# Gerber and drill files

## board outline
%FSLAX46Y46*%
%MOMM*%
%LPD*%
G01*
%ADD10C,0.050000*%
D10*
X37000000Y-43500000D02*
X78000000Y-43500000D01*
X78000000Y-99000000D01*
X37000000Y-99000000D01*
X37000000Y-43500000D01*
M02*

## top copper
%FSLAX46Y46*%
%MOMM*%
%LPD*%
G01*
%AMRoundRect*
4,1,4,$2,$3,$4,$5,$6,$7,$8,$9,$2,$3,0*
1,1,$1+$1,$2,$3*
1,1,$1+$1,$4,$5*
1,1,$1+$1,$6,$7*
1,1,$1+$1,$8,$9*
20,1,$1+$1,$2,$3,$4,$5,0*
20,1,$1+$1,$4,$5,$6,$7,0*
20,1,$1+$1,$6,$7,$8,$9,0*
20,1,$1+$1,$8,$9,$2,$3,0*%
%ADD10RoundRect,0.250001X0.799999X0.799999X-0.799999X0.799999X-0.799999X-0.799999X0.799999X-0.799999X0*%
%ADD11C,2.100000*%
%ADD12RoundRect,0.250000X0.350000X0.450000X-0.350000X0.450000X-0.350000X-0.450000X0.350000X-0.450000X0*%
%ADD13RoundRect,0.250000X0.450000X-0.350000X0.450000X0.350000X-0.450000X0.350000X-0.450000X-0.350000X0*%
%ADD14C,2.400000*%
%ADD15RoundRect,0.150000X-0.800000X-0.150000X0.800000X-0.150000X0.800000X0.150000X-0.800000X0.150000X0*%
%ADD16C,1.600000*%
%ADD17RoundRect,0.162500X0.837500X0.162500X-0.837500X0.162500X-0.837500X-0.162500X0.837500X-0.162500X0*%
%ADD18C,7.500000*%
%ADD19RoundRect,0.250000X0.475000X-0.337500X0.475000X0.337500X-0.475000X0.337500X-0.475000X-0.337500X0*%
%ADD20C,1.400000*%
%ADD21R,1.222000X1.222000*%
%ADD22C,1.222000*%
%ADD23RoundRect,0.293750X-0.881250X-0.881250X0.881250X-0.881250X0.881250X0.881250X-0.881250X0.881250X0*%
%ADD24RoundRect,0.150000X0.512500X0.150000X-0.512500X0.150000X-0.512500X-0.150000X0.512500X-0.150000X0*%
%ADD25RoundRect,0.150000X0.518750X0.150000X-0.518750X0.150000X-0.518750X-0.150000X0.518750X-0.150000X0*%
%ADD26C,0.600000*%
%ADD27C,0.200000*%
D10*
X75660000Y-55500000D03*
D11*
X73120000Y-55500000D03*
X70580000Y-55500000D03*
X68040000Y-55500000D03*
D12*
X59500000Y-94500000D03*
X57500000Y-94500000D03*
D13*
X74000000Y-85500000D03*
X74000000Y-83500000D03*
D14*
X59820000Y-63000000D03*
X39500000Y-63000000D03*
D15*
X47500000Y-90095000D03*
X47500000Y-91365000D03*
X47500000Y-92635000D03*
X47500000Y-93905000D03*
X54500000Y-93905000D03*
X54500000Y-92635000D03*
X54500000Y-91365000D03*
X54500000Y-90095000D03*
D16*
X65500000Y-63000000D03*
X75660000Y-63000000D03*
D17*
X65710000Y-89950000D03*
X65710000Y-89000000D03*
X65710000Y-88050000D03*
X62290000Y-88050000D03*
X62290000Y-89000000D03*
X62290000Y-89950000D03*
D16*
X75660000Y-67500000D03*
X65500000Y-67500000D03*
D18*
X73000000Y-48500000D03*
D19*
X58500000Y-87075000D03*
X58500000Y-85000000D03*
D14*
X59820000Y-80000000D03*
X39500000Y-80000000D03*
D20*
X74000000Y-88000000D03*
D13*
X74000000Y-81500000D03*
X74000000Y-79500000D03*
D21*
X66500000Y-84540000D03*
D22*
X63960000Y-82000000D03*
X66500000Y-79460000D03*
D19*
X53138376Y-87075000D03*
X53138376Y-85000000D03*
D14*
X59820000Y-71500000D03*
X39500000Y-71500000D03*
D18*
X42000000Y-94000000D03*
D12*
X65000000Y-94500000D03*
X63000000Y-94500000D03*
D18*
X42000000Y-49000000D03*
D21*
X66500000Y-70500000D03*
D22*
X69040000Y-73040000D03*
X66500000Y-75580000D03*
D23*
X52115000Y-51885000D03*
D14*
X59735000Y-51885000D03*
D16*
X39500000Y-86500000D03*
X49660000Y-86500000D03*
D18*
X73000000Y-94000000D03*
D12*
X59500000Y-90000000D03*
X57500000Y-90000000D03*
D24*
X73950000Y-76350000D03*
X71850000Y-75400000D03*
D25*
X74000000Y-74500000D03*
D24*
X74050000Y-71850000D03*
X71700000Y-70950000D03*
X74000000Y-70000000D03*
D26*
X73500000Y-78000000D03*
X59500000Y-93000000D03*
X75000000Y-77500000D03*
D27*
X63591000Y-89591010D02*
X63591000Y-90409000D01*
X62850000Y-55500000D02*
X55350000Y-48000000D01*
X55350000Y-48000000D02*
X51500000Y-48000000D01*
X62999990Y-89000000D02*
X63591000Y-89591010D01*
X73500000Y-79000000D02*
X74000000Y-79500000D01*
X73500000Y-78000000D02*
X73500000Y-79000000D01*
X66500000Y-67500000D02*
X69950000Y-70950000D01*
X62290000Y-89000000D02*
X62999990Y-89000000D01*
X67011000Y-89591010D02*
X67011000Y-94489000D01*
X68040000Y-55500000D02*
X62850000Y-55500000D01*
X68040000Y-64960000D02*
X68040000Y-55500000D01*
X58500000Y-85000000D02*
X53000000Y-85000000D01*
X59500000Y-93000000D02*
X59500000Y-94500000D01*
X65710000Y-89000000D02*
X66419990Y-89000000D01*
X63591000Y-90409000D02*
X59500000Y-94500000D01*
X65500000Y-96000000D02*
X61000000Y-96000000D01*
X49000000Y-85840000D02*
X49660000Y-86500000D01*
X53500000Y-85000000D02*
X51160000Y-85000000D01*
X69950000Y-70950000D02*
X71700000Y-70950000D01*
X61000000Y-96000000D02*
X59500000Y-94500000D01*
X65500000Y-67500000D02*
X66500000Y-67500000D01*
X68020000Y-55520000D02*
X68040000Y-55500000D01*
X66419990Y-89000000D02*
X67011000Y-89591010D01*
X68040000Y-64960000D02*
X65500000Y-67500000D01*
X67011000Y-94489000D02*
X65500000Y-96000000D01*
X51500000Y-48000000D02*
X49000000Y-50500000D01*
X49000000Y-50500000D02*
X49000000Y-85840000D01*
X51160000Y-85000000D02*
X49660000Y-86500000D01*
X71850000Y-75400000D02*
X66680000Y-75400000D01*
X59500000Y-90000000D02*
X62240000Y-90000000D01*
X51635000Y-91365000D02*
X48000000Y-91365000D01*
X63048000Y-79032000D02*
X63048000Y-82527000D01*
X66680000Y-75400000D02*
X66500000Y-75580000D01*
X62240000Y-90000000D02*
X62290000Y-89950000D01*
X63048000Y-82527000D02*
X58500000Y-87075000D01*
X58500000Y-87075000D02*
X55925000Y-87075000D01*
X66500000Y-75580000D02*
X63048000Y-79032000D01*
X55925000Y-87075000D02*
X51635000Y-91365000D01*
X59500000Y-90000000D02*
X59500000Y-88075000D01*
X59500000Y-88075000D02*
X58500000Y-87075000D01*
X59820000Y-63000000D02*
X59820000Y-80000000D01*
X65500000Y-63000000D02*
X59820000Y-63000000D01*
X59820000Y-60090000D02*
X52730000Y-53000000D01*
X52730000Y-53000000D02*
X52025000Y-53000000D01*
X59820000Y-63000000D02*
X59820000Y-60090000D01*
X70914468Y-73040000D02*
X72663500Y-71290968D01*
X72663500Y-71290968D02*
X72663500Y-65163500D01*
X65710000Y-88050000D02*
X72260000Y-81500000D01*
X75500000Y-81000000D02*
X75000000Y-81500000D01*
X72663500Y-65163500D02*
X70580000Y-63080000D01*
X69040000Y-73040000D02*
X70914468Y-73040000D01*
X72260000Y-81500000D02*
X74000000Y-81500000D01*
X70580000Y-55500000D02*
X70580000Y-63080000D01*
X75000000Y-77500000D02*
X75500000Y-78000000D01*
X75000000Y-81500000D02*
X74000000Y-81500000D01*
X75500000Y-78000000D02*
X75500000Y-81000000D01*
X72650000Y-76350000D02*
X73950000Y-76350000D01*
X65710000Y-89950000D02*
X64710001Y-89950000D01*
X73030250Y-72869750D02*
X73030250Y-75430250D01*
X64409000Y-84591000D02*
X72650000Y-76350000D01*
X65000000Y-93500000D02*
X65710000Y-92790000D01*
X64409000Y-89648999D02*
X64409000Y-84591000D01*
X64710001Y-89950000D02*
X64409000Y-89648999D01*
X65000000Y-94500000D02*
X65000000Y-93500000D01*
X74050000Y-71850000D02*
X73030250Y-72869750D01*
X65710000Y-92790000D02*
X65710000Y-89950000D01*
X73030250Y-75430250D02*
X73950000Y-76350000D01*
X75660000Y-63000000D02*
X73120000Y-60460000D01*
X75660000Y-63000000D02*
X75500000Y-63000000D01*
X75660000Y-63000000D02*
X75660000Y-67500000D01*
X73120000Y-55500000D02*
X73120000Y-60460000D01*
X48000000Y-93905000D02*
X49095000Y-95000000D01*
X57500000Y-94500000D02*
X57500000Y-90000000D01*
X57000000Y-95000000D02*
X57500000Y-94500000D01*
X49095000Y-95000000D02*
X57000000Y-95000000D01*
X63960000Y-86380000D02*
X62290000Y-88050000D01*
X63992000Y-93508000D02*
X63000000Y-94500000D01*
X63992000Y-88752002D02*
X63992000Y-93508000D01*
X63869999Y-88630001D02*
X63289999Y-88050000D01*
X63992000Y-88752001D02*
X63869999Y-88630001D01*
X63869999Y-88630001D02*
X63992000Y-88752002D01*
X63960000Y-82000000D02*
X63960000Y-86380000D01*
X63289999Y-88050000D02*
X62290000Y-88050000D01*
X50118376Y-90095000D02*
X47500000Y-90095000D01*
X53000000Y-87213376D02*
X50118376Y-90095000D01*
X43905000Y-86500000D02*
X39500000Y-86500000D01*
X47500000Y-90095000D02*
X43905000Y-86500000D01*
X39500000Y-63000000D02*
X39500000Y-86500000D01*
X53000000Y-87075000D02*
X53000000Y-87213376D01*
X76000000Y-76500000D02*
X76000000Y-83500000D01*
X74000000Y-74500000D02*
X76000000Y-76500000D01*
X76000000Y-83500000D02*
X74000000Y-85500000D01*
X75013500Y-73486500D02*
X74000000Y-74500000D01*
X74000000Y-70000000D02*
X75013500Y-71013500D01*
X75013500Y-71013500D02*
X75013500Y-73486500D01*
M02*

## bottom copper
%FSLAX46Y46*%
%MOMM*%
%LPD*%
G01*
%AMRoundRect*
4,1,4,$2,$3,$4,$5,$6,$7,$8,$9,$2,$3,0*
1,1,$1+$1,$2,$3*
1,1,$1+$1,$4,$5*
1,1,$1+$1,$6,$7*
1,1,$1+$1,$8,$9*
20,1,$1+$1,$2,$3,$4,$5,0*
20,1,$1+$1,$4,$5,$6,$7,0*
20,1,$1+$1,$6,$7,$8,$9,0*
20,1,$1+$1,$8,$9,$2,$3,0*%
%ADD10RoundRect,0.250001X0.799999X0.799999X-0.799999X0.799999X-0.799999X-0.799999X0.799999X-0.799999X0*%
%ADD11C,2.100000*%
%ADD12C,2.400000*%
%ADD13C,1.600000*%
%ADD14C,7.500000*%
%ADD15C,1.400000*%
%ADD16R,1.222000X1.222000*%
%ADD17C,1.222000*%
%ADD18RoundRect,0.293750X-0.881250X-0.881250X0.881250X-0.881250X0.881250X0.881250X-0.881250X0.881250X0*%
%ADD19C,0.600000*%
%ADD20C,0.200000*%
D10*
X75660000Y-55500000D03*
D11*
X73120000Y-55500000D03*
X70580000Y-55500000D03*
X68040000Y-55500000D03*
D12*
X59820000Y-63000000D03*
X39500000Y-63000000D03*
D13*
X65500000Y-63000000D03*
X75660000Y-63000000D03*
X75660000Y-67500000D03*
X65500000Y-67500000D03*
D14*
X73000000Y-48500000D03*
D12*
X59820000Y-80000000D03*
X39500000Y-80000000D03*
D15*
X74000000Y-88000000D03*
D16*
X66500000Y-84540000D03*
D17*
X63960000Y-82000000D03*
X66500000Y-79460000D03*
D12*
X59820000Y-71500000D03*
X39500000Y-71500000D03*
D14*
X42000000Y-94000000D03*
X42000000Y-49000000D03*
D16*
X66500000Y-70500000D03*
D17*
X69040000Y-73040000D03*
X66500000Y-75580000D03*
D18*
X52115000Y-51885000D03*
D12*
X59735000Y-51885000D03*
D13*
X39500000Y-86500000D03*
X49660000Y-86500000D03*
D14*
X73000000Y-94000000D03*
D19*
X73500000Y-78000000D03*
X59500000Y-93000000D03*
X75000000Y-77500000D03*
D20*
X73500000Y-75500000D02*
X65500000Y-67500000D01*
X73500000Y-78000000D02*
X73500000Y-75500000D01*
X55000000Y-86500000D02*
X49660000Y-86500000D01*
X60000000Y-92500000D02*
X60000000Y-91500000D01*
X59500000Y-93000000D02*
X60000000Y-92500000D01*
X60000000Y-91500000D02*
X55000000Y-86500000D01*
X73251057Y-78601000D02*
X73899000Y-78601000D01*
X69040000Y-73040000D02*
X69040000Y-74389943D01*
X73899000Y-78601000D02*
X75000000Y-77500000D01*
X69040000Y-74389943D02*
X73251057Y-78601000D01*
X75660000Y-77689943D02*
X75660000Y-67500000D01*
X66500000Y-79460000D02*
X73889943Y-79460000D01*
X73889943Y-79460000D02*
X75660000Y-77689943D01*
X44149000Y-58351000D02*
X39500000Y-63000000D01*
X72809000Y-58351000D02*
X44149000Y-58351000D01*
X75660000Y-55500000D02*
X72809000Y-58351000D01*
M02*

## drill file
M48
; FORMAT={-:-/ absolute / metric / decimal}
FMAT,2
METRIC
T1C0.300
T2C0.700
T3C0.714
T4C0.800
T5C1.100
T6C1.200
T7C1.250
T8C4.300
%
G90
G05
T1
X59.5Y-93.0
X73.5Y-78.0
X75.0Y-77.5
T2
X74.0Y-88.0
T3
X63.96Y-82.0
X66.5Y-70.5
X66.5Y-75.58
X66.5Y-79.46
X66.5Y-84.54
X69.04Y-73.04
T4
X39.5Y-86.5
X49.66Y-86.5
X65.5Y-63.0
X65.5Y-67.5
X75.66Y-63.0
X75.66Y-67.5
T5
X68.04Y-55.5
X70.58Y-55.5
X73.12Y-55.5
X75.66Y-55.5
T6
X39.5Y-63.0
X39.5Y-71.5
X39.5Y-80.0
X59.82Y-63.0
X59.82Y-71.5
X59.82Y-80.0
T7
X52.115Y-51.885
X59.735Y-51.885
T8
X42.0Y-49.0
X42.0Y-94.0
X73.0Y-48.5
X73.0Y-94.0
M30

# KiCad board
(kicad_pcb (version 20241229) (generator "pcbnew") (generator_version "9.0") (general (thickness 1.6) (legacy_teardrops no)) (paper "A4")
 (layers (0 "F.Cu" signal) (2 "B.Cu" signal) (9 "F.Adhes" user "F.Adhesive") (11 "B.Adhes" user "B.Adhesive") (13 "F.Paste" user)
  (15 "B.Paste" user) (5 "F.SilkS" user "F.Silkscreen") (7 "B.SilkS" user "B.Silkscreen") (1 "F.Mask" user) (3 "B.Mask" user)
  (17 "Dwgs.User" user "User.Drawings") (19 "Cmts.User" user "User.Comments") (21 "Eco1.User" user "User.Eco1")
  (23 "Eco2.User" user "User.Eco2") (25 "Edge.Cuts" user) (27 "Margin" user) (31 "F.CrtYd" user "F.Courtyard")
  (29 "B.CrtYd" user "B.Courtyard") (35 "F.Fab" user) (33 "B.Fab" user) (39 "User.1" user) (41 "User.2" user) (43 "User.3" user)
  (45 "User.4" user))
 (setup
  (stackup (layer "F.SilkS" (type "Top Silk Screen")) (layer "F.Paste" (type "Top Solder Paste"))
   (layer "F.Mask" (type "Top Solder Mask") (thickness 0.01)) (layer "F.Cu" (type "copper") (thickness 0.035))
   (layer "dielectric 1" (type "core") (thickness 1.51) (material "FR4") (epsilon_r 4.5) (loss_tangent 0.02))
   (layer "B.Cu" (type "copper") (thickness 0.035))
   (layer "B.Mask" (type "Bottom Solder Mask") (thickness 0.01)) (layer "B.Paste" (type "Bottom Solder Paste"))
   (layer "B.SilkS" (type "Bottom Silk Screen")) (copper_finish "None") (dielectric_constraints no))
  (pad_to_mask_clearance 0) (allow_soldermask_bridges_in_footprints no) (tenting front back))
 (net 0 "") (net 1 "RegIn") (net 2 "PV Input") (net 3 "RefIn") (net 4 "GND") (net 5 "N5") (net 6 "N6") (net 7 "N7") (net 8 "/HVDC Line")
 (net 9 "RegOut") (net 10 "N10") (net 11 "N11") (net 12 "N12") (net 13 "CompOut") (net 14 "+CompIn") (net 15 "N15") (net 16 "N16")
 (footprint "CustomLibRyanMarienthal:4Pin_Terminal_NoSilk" (layer "F.Cu") (at 71.85 55.54 180)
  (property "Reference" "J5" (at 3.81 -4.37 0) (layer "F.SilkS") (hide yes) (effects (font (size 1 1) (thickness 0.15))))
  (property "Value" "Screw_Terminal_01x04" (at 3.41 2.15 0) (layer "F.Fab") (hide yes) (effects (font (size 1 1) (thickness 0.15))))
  (pad "1" thru_hole roundrect (at -3.81 0.04 180) (size 2.1 2.1) (drill 1.1) (layers "*.Cu" "*.Mask") (remove_unused_layers no)
   (roundrect_rratio 0.119048) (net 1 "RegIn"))
  (pad "2" thru_hole circle (at -1.27 0.04 180) (size 2.1 2.1) (drill 1.1) (layers "*.Cu" "*.Mask") (remove_unused_layers no)
   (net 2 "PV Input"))
  (pad "3" thru_hole circle (at 1.27 0.04 180) (size 2.1 2.1) (drill 1.1) (layers "*.Cu" "*.Mask") (remove_unused_layers no) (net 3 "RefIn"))
  (pad "4" thru_hole circle (at 3.81 0.04 180) (size 2.1 2.1) (drill 1.1) (layers "*.Cu" "*.Mask") (remove_unused_layers no) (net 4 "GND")))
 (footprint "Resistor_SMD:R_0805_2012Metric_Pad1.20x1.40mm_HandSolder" (layer "F.Cu") (at 58.5 94.5 180)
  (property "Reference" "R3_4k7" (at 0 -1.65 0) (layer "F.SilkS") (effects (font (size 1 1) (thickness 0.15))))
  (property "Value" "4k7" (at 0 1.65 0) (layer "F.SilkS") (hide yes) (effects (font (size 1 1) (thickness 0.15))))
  (pad "1" smd roundrect (at -1 0 180) (size 1.2 1.4) (layers "F.Cu" "F.Mask" "F.Paste") (roundrect_rratio 0.208333) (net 4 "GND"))
  (pad "2" smd roundrect (at 1 0 180) (size 1.2 1.4) (layers "F.Cu" "F.Mask" "F.Paste") (roundrect_rratio 0.208333) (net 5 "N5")))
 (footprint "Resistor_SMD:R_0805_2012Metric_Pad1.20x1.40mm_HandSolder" (layer "F.Cu") (at 74 84.5 90)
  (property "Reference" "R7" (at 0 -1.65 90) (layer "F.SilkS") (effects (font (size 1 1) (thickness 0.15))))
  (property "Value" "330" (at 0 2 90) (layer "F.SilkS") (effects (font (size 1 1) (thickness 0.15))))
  (pad "1" smd roundrect (at -1 0 90) (size 1.2 1.4) (layers "F.Cu" "F.Mask" "F.Paste") (roundrect_rratio 0.208333) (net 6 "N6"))
  (pad "2" smd roundrect (at 1 0 90) (size 1.2 1.4) (layers "F.Cu" "F.Mask" "F.Paste") (roundrect_rratio 0.208333) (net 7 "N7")))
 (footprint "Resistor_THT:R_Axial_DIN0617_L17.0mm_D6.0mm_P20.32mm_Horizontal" (layer "F.Cu") (at 59.82 63 180)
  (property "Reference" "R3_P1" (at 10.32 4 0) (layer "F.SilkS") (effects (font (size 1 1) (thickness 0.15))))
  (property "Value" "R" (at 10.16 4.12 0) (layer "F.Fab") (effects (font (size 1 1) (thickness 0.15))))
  (pad "1" thru_hole circle (at 0 0 180) (size 2.4 2.4) (drill 1.2) (layers "*.Cu" "*.Mask") (remove_unused_layers no) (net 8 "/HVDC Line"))
  (pad "2" thru_hole circle (at 20.32 0 180) (size 2.4 2.4) (drill 1.2) (layers "*.Cu" "*.Mask") (remove_unused_layers no) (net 1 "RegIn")))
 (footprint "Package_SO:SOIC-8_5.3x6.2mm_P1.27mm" (layer "F.Cu") (at 51 92)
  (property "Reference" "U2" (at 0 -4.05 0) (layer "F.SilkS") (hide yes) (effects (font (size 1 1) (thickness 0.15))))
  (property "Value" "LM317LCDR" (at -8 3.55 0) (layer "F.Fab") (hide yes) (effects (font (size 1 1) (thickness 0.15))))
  (pad "1" smd roundrect (at -3.5 -1.905) (size 1.9 0.6) (layers "F.Cu" "F.Mask" "F.Paste") (roundrect_rratio 0.25) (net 1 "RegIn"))
  (pad "2" smd roundrect (at -3.5 -0.635) (size 1.9 0.6) (layers "F.Cu" "F.Mask" "F.Paste") (roundrect_rratio 0.25) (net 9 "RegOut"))
  (pad "3" smd roundrect (at -3.5 0.635) (size 1.9 0.6) (layers "F.Cu" "F.Mask" "F.Paste") (roundrect_rratio 0.25) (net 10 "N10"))
  (pad "4" smd roundrect (at -3.5 1.905) (size 1.9 0.6) (layers "F.Cu" "F.Mask" "F.Paste") (roundrect_rratio 0.25) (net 5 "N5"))
  (pad "5" smd roundrect (at 3.5 1.905) (size 1.9 0.6) (layers "F.Cu" "F.Mask" "F.Paste") (roundrect_rratio 0.25))
  (pad "6" smd roundrect (at 3.5 0.635) (size 1.9 0.6) (layers "F.Cu" "F.Mask" "F.Paste") (roundrect_rratio 0.25) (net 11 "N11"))
  (pad "7" smd roundrect (at 3.5 -0.635) (size 1.9 0.6) (layers "F.Cu" "F.Mask" "F.Paste") (roundrect_rratio 0.25) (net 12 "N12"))
  (pad "8" smd roundrect (at 3.5 -1.905) (size 1.9 0.6) (layers "F.Cu" "F.Mask" "F.Paste") (roundrect_rratio 0.25)))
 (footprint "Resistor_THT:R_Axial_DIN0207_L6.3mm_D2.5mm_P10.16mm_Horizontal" (layer "F.Cu") (at 65.5 63)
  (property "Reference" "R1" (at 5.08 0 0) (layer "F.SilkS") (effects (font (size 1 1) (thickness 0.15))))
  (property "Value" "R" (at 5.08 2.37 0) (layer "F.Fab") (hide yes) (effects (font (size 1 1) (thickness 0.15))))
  (pad "1" thru_hole circle (at 0 0) (size 1.6 1.6) (drill 0.8) (layers "*.Cu" "*.Mask") (remove_unused_layers no) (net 8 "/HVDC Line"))
  (pad "2" thru_hole circle (at 10.16 0) (size 1.6 1.6) (drill 0.8) (layers "*.Cu" "*.Mask") (remove_unused_layers no) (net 2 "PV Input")))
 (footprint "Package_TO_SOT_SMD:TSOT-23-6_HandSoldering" (layer "F.Cu") (at 64 89 180)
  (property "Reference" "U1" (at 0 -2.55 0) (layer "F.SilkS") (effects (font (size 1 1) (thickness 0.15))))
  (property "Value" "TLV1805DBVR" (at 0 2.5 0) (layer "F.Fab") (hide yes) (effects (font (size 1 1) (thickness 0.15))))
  (pad "1" smd roundrect (at -1.71 -0.95 180) (size 2 0.65) (layers "F.Cu" "F.Mask" "F.Paste") (roundrect_rratio 0.25) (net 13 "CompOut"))
  (pad "2" smd roundrect (at -1.71 0 180) (size 2 0.65) (layers "F.Cu" "F.Mask" "F.Paste") (roundrect_rratio 0.25) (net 4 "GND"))
  (pad "3" smd roundrect (at -1.71 0.95 180) (size 2 0.65) (layers "F.Cu" "F.Mask" "F.Paste") (roundrect_rratio 0.25) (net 3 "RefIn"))
  (pad "4" smd roundrect (at 1.71 0.95 180) (size 2 0.65) (layers "F.Cu" "F.Mask" "F.Paste") (roundrect_rratio 0.25) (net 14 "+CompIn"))
  (pad "5" smd roundrect (at 1.71 0 180) (size 2 0.65) (layers "F.Cu" "F.Mask" "F.Paste") (roundrect_rratio 0.25) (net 4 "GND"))
  (pad "6" smd roundrect (at 1.71 -0.95 180) (size 2 0.65) (layers "F.Cu" "F.Mask" "F.Paste") (roundrect_rratio 0.25) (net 9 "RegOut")))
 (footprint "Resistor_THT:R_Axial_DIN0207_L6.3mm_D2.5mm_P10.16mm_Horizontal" (layer "F.Cu") (at 75.66 67.5 180)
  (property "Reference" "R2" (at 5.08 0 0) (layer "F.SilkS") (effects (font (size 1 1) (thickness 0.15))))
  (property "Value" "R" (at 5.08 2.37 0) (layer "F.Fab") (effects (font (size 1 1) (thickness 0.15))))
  (pad "1" thru_hole circle (at 0 0 180) (size 1.6 1.6) (drill 0.8) (layers "*.Cu" "*.Mask") (remove_unused_layers no) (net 2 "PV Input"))
  (pad "2" thru_hole circle (at 10.16 0 180) (size 1.6 1.6) (drill 0.8) (layers "*.Cu" "*.Mask") (remove_unused_layers no) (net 4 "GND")))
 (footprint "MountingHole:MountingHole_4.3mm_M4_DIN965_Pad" (layer "F.Cu") (at 73 48.5)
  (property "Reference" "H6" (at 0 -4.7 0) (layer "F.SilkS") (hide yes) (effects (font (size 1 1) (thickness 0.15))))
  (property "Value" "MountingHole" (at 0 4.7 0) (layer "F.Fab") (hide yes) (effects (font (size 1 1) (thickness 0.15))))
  (pad "1" thru_hole circle (at 0 0) (size 7.5 7.5) (drill 4.3) (layers "*.Cu" "*.Mask") (remove_unused_layers no) (zone_connect 2)))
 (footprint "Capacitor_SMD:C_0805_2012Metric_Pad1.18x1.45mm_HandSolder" (layer "F.Cu") (at 58.5 86.0375 90)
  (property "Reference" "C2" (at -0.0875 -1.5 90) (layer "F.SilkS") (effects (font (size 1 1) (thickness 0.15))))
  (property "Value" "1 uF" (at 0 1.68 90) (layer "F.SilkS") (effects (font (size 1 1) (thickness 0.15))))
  (pad "1" smd roundrect (at -1.0375 0 90) (size 1.175 1.45) (layers "F.Cu" "F.Mask" "F.Paste") (roundrect_rratio 0.212766) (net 9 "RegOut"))
  (pad "2" smd roundrect (at 1.0375 0 90) (size 1.175 1.45) (layers "F.Cu" "F.Mask" "F.Paste") (roundrect_rratio 0.212766) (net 4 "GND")))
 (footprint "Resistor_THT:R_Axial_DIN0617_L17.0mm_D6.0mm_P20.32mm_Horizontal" (layer "F.Cu") (at 59.82 80 180)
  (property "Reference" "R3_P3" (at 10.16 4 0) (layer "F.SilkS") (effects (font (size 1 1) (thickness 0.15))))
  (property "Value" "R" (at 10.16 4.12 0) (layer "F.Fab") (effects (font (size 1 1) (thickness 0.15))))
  (pad "1" thru_hole circle (at 0 0 180) (size 2.4 2.4) (drill 1.2) (layers "*.Cu" "*.Mask") (remove_unused_layers no) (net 8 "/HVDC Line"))
  (pad "2" thru_hole circle (at 20.32 0 180) (size 2.4 2.4) (drill 1.2) (layers "*.Cu" "*.Mask") (remove_unused_layers no) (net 1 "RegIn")))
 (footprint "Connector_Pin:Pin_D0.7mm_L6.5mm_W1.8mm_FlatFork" (layer "F.Cu") (at 74 88)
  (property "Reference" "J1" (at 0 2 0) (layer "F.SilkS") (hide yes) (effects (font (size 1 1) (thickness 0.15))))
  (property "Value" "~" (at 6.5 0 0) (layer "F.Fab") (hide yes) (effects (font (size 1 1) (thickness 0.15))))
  (pad "1" thru_hole circle (at 0 0) (size 1.4 1.4) (drill 0.7) (layers "*.Cu" "*.Mask") (remove_unused_layers no) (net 7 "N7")))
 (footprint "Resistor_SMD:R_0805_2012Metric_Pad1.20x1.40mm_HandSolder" (layer "F.Cu") (at 74 80.5 90)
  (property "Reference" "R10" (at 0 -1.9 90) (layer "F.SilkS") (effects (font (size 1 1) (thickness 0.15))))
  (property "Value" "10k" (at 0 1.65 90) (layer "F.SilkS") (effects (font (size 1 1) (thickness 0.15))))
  (pad "1" smd roundrect (at -1 0 90) (size 1.2 1.4) (layers "F.Cu" "F.Mask" "F.Paste") (roundrect_rratio 0.208333) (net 3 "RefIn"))
  (pad "2" smd roundrect (at 1 0 90) (size 1.2 1.4) (layers "F.Cu" "F.Mask" "F.Paste") (roundrect_rratio 0.208333) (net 4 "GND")))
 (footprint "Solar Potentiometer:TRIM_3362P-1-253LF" (layer "F.Cu") (at 66.5 82 90)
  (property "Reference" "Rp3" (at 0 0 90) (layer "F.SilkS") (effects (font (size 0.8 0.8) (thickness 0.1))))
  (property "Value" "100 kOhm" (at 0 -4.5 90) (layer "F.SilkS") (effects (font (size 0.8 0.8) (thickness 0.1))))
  (pad "1" thru_hole rect (at -2.54 0 90) (size 1.222 1.222) (drill 0.714) (layers "*.Cu" "*.Mask") (remove_unused_layers no) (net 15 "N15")
   (solder_mask_margin 0.102))
  (pad "2" thru_hole circle (at 0 -2.54 90) (size 1.222 1.222) (drill 0.714) (layers "*.Cu" "*.Mask") (remove_unused_layers no)
   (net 14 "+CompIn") (solder_mask_margin 0.102))
  (pad "3" thru_hole circle (at 2.54 0 90) (size 1.222 1.222) (drill 0.714) (layers "*.Cu" "*.Mask") (remove_unused_layers no)
   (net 2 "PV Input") (solder_mask_margin 0.102)))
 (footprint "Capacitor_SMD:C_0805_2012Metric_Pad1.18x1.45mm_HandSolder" (layer "F.Cu") (at 53.138376 86.0375 90)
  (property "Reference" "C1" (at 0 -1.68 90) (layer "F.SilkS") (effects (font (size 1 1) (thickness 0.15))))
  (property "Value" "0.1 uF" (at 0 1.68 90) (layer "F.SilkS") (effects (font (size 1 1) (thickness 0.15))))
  (pad "1" smd roundrect (at -1.0375 0 90) (size 1.175 1.45) (layers "F.Cu" "F.Mask" "F.Paste") (roundrect_rratio 0.212766) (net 1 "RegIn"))
  (pad "2" smd roundrect (at 1.0375 0 90) (size 1.175 1.45) (layers "F.Cu" "F.Mask" "F.Paste") (roundrect_rratio 0.212766) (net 4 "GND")))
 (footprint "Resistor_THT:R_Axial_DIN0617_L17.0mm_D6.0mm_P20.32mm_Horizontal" (layer "F.Cu") (at 59.82 71.5 180)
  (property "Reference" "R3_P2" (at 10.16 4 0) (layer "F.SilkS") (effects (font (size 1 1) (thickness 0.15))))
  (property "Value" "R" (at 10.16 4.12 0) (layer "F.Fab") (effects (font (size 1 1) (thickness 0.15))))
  (pad "1" thru_hole circle (at 0 0 180) (size 2.4 2.4) (drill 1.2) (layers "*.Cu" "*.Mask") (remove_unused_layers no) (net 8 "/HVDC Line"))
  (pad "2" thru_hole circle (at 20.32 0 180) (size 2.4 2.4) (drill 1.2) (layers "*.Cu" "*.Mask") (remove_unused_layers no) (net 1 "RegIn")))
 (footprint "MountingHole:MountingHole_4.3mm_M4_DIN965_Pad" (layer "F.Cu") (at 42 94)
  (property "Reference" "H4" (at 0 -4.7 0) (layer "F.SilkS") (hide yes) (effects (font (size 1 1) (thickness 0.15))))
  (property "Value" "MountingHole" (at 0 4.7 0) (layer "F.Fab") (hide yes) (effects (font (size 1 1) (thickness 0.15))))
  (pad "1" thru_hole circle (at 0 0) (size 7.5 7.5) (drill 4.3) (layers "*.Cu" "*.Mask") (remove_unused_layers no) (zone_connect 2)))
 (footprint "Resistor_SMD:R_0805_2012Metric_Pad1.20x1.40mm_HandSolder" (layer "F.Cu") (at 64 94.5 180)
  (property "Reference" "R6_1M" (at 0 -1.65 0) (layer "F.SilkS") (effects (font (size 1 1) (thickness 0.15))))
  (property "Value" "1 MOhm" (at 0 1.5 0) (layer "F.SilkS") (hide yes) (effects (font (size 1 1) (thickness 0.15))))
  (pad "1" smd roundrect (at -1 0 180) (size 1.2 1.4) (layers "F.Cu" "F.Mask" "F.Paste") (roundrect_rratio 0.208333) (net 13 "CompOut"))
  (pad "2" smd roundrect (at 1 0 180) (size 1.2 1.4) (layers "F.Cu" "F.Mask" "F.Paste") (roundrect_rratio 0.208333) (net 14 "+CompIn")))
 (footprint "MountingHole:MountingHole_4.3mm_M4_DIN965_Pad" (layer "F.Cu") (at 42 49)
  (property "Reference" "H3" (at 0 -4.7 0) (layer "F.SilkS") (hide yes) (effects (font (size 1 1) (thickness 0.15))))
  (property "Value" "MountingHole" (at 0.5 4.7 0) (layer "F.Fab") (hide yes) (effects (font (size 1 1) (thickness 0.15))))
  (pad "1" thru_hole circle (at 0 0) (size 7.5 7.5) (drill 4.3) (layers "*.Cu" "*.Mask") (remove_unused_layers no) (zone_connect 2)))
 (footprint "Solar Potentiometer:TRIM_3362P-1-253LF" (layer "F.Cu") (at 66.5 73.04 -90)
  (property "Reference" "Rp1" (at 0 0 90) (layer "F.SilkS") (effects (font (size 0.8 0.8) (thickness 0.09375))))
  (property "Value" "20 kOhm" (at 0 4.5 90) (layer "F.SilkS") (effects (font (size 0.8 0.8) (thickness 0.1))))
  (pad "1" thru_hole rect (at -2.54 0 270) (size 1.222 1.222) (drill 0.714) (layers "*.Cu" "*.Mask") (remove_unused_layers no)
   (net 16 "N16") (solder_mask_margin 0.102))
  (pad "2" thru_hole circle (at 0 -2.54 270) (size 1.222 1.222) (drill 0.714) (layers "*.Cu" "*.Mask") (remove_unused_layers no)
   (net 3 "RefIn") (solder_mask_margin 0.102))
  (pad "3" thru_hole circle (at 2.54 0 270) (size 1.222 1.222) (drill 0.714) (layers "*.Cu" "*.Mask") (remove_unused_layers no)
   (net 9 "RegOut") (solder_mask_margin 0.102)))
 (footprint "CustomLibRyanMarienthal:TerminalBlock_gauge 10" (layer "F.Cu") (at 48.025 56.435)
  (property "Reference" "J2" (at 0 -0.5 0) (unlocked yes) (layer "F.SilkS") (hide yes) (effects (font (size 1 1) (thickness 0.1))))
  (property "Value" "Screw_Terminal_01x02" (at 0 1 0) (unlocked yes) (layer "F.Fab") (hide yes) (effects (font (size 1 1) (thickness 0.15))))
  (pad "1" thru_hole roundrect (at 4.09 -4.55) (size 2.35 2.35) (drill 1.25) (layers "*.Cu" "*.Mask") (remove_unused_layers no)
   (roundrect_rratio 0.125) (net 8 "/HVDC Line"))
  (pad "2" thru_hole circle (at 11.71 -4.55) (size 2.4 2.4) (drill 1.25) (layers "*.Cu" "*.Mask") (remove_unused_layers no) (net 4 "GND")))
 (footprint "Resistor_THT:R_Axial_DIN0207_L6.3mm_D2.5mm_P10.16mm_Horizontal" (layer "F.Cu") (at 39.5 86.5)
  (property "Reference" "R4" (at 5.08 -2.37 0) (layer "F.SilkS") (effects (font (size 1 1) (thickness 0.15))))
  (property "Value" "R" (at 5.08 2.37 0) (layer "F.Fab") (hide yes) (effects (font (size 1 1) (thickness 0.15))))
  (pad "1" thru_hole circle (at 0 0) (size 1.6 1.6) (drill 0.8) (layers "*.Cu" "*.Mask") (remove_unused_layers no) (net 1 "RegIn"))
  (pad "2" thru_hole circle (at 10.16 0) (size 1.6 1.6) (drill 0.8) (layers "*.Cu" "*.Mask") (remove_unused_layers no) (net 4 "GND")))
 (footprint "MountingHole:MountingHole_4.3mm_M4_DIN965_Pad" (layer "F.Cu") (at 73 94)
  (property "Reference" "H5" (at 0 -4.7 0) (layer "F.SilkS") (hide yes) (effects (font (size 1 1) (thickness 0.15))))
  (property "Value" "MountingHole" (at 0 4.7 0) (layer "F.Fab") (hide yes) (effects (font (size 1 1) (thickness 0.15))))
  (pad "1" thru_hole circle (at 0 0) (size 7.5 7.5) (drill 4.3) (layers "*.Cu" "*.Mask") (remove_unused_layers no) (zone_connect 2)))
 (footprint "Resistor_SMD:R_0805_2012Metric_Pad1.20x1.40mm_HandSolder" (layer "F.Cu") (at 58.5 90 180)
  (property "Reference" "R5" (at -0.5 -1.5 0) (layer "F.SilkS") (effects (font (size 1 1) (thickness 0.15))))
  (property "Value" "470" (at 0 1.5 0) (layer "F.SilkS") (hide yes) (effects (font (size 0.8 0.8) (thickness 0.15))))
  (pad "1" smd roundrect (at -1 0 180) (size 1.2 1.4) (layers "F.Cu" "F.Mask" "F.Paste") (roundrect_rratio 0.208333) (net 9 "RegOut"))
  (pad "2" smd roundrect (at 1 0 180) (size 1.2 1.4) (layers "F.Cu" "F.Mask" "F.Paste") (roundrect_rratio 0.208333) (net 5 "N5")))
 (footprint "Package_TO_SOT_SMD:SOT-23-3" (layer "F.Cu") (at 72.8 75.4 180)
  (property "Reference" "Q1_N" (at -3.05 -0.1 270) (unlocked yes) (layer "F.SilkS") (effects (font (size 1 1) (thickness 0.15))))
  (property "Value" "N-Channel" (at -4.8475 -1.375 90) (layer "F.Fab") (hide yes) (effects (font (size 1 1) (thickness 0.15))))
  (pad "1" smd roundrect (at -1.15 -0.95 180) (size 1.325 0.6) (layers "F.Cu" "F.Mask" "F.Paste") (roundrect_rratio 0.25) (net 13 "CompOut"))
  (pad "2" smd roundrect (at 0.95 0 180) (size 1.325 0.6) (layers "F.Cu" "F.Mask" "F.Paste") (roundrect_rratio 0.25) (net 9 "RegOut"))
  (pad "3" smd roundrect (at -1.2 0.9 180) (size 1.3375 0.6) (layers "F.Cu" "F.Mask" "F.Paste") (roundrect_rratio 0.25) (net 6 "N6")))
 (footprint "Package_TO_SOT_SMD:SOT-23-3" (layer "F.Cu") (at 72.85 70.95 180)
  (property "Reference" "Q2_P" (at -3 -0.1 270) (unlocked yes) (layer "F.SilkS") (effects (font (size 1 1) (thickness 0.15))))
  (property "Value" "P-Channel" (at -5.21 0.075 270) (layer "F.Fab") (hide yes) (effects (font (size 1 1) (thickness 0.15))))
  (pad "1" smd roundrect (at -1.2 -0.9 180) (size 1.325 0.6) (layers "F.Cu" "F.Mask" "F.Paste") (roundrect_rratio 0.25) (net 13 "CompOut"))
  (pad "2" smd roundrect (at 1.15 0 180) (size 1.325 0.6) (layers "F.Cu" "F.Mask" "F.Paste") (roundrect_rratio 0.25) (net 4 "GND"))
  (pad "3" smd roundrect (at -1.15 0.95 180) (size 1.325 0.6) (layers "F.Cu" "F.Mask" "F.Paste") (roundrect_rratio 0.25) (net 6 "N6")))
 (gr_rect (start 37 43.5) (end 78 99) (stroke (width 0.05) (type default)) (fill no) (layer "Edge.Cuts"))
 (segment (start 63.591 89.59101) (end 63.591 90.409) (width 0.2) (layer "F.Cu") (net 4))
 (segment (start 62.85 55.5) (end 55.35 48) (width 0.2) (layer "F.Cu") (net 4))
 (segment (start 55.35 48) (end 51.5 48) (width 0.2) (layer "F.Cu") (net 4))
 (segment (start 62.99999 89) (end 63.591 89.59101) (width 0.2) (layer "F.Cu") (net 4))
 (segment (start 73.5 79) (end 74 79.5) (width 0.2) (layer "F.Cu") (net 4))
 (segment (start 73.5 78) (end 73.5 79) (width 0.2) (layer "F.Cu") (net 4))
 (segment (start 66.5 67.5) (end 69.95 70.95) (width 0.2) (layer "F.Cu") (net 4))
 (segment (start 62.29 89) (end 62.99999 89) (width 0.2) (layer "F.Cu") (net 4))
 (segment (start 67.011 89.59101) (end 67.011 94.489) (width 0.2) (layer "F.Cu") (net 4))
 (segment (start 68.04 55.5) (end 62.85 55.5) (width 0.2) (layer "F.Cu") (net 4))
 (segment (start 68.04 64.96) (end 68.04 55.5) (width 0.2) (layer "F.Cu") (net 4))
 (segment (start 58.5 85) (end 53 85) (width 0.2) (layer "F.Cu") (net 4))
 (segment (start 59.5 93) (end 59.5 94.5) (width 0.2) (layer "F.Cu") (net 4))
 (segment (start 65.71 89) (end 66.41999 89) (width 0.2) (layer "F.Cu") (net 4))
 (segment (start 63.591 90.409) (end 59.5 94.5) (width 0.2) (layer "F.Cu") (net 4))
 (segment (start 65.5 96) (end 61 96) (width 0.2) (layer "F.Cu") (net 4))
 (segment (start 49 85.84) (end 49.66 86.5) (width 0.2) (layer "F.Cu") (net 4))
 (segment (start 53.5 85) (end 51.16 85) (width 0.2) (layer "F.Cu") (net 4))
 (segment (start 69.95 70.95) (end 71.7 70.95) (width 0.2) (layer "F.Cu") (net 4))
 (segment (start 61 96) (end 59.5 94.5) (width 0.2) (layer "F.Cu") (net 4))
 (segment (start 65.5 67.5) (end 66.5 67.5) (width 0.2) (layer "F.Cu") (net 4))
 (segment (start 68.02 55.52) (end 68.04 55.5) (width 0.2) (layer "F.Cu") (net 4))
 (segment (start 66.41999 89) (end 67.011 89.59101) (width 0.2) (layer "F.Cu") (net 4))
 (segment (start 68.04 64.96) (end 65.5 67.5) (width 0.2) (layer "F.Cu") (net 4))
 (segment (start 67.011 94.489) (end 65.5 96) (width 0.2) (layer "F.Cu") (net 4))
 (segment (start 51.5 48) (end 49 50.5) (width 0.2) (layer "F.Cu") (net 4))
 (segment (start 49 50.5) (end 49 85.84) (width 0.2) (layer "F.Cu") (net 4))
 (segment (start 51.16 85) (end 49.66 86.5) (width 0.2) (layer "F.Cu") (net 4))
 (via (at 73.5 78) (size 0.6) (drill 0.3) (layers "F.Cu" "B.Cu") (free yes) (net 4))
 (via (at 59.5 93) (size 0.6) (drill 0.3) (layers "F.Cu" "B.Cu") (free yes) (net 4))
 (segment (start 73.5 75.5) (end 65.5 67.5) (width 0.2) (layer "B.Cu") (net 4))
 (segment (start 73.5 78) (end 73.5 75.5) (width 0.2) (layer "B.Cu") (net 4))
 (segment (start 55 86.5) (end 49.66 86.5) (width 0.2) (layer "B.Cu") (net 4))
 (segment (start 60 92.5) (end 60 91.5) (width 0.2) (layer "B.Cu") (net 4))
 (segment (start 59.5 93) (end 60 92.5) (width 0.2) (layer "B.Cu") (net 4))
 (segment (start 60 91.5) (end 55 86.5) (width 0.2) (layer "B.Cu") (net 4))
 (segment (start 71.85 75.4) (end 66.68 75.4) (width 0.2) (layer "F.Cu") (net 9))
 (segment (start 59.5 90) (end 62.24 90) (width 0.2) (layer "F.Cu") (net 9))
 (segment (start 51.635 91.365) (end 48 91.365) (width 0.2) (layer "F.Cu") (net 9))
 (segment (start 63.048 79.032) (end 63.048 82.527) (width 0.2) (layer "F.Cu") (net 9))
 (segment (start 66.68 75.4) (end 66.5 75.58) (width 0.2) (layer "F.Cu") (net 9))
 (segment (start 62.24 90) (end 62.29 89.95) (width 0.2) (layer "F.Cu") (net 9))
 (segment (start 63.048 82.527) (end 58.5 87.075) (width 0.2) (layer "F.Cu") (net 9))
 (segment (start 58.5 87.075) (end 55.925 87.075) (width 0.2) (layer "F.Cu") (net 9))
 (segment (start 66.5 75.58) (end 63.048 79.032) (width 0.2) (layer "F.Cu") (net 9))
 (segment (start 55.925 87.075) (end 51.635 91.365) (width 0.2) (layer "F.Cu") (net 9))
 (segment (start 59.5 90) (end 59.5 88.075) (width 0.2) (layer "F.Cu") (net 9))
 (segment (start 59.5 88.075) (end 58.5 87.075) (width 0.2) (layer "F.Cu") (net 9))
 (segment (start 59.82 63) (end 59.82 80) (width 0.2) (layer "F.Cu") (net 8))
 (segment (start 65.5 63) (end 59.82 63) (width 0.2) (layer "F.Cu") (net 8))
 (segment (start 59.82 60.09) (end 52.73 53) (width 0.2) (layer "F.Cu") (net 8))
 (segment (start 52.73 53) (end 52.025 53) (width 0.2) (layer "F.Cu") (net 8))
 (segment (start 59.82 63) (end 59.82 60.09) (width 0.2) (layer "F.Cu") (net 8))
 (segment (start 70.914468 73.04) (end 72.6635 71.290968) (width 0.2) (layer "F.Cu") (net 3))
 (segment (start 72.6635 71.290968) (end 72.6635 65.1635) (width 0.2) (layer "F.Cu") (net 3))
 (segment (start 65.71 88.05) (end 72.26 81.5) (width 0.2) (layer "F.Cu") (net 3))
 (segment (start 75.5 81) (end 75 81.5) (width 0.2) (layer "F.Cu") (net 3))
 (segment (start 72.6635 65.1635) (end 70.58 63.08) (width 0.2) (layer "F.Cu") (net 3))
 (segment (start 69.04 73.04) (end 70.914468 73.04) (width 0.2) (layer "F.Cu") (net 3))
 (segment (start 72.26 81.5) (end 74 81.5) (width 0.2) (layer "F.Cu") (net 3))
 (segment (start 70.58 55.5) (end 70.58 63.08) (width 0.2) (layer "F.Cu") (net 3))
 (segment (start 75 77.5) (end 75.5 78) (width 0.2) (layer "F.Cu") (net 3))
 (segment (start 75 81.5) (end 74 81.5) (width 0.2) (layer "F.Cu") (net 3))
 (segment (start 75.5 78) (end 75.5 81) (width 0.2) (layer "F.Cu") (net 3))
 (via (at 75 77.5) (size 0.6) (drill 0.3) (layers "F.Cu" "B.Cu") (free yes) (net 3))
 (segment (start 73.251057 78.601) (end 73.899 78.601) (width 0.2) (layer "B.Cu") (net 3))
 (segment (start 69.04 73.04) (end 69.04 74.389943) (width 0.2) (layer "B.Cu") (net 3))
 (segment (start 73.899 78.601) (end 75 77.5) (width 0.2) (layer "B.Cu") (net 3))
 (segment (start 69.04 74.389943) (end 73.251057 78.601) (width 0.2) (layer "B.Cu") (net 3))
 (segment (start 72.65 76.35) (end 73.95 76.35) (width 0.2) (layer "F.Cu") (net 13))
 (segment (start 65.71 89.95) (end 64.710001 89.95) (width 0.2) (layer "F.Cu") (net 13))
 (segment (start 73.03025 72.86975) (end 73.03025 75.43025) (width 0.2) (layer "F.Cu") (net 13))
 (segment (start 64.409 84.591) (end 72.65 76.35) (width 0.2) (layer "F.Cu") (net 13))
 (segment (start 65 93.5) (end 65.71 92.79) (width 0.2) (layer "F.Cu") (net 13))
 (segment (start 64.409 89.648999) (end 64.409 84.591) (width 0.2) (layer "F.Cu") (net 13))
 (segment (start 64.710001 89.95) (end 64.409 89.648999) (width 0.2) (layer "F.Cu") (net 13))
 (segment (start 65 94.5) (end 65 93.5) (width 0.2) (layer "F.Cu") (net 13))
 (segment (start 74.05 71.85) (end 73.03025 72.86975) (width 0.2) (layer "F.Cu") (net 13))
 (segment (start 65.71 92.79) (end 65.71 89.95) (width 0.2) (layer "F.Cu") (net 13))
 (segment (start 73.03025 75.43025) (end 73.95 76.35) (width 0.2) (layer "F.Cu") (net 13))
 (segment (start 75.66 63) (end 73.12 60.46) (width 0.2) (layer "F.Cu") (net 2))
 (segment (start 75.66 63) (end 75.5 63) (width 0.2) (layer "F.Cu") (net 2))
 (segment (start 75.66 63) (end 75.66 67.5) (width 0.2) (layer "F.Cu") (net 2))
 (segment (start 73.12 55.5) (end 73.12 60.46) (width 0.2) (layer "F.Cu") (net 2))
 (segment (start 75.66 77.689943) (end 75.66 67.5) (width 0.2) (layer "B.Cu") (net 2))
 (segment (start 66.5 79.46) (end 73.889943 79.46) (width 0.2) (layer "B.Cu") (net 2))
 (segment (start 73.889943 79.46) (end 75.66 77.689943) (width 0.2) (layer "B.Cu") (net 2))
 (segment (start 48 93.905) (end 49.095 95) (width 0.2) (layer "F.Cu") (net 5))
 (segment (start 57.5 94.5) (end 57.5 90) (width 0.2) (layer "F.Cu") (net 5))
 (segment (start 57 95) (end 57.5 94.5) (width 0.2) (layer "F.Cu") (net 5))
 (segment (start 49.095 95) (end 57 95) (width 0.2) (layer "F.Cu") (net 5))
 (segment (start 63.96 86.38) (end 62.29 88.05) (width 0.2) (layer "F.Cu") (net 14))
 (segment (start 63.992 93.508) (end 63 94.5) (width 0.2) (layer "F.Cu") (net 14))
 (segment (start 63.992 88.752002) (end 63.992 93.508) (width 0.2) (layer "F.Cu") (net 14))
 (segment (start 63.869999 88.630001) (end 63.289999 88.05) (width 0.2) (layer "F.Cu") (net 14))
 (segment (start 63.992 88.752001) (end 63.869999 88.630001) (width 0.2) (layer "F.Cu") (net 14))
 (segment (start 63.869999 88.630001) (end 63.992 88.752002) (width 0.2) (layer "F.Cu") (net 14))
 (segment (start 63.96 82) (end 63.96 86.38) (width 0.2) (layer "F.Cu") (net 14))
 (segment (start 63.289999 88.05) (end 62.29 88.05) (width 0.2) (layer "F.Cu") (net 14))
 (segment (start 50.118376 90.095) (end 47.5 90.095) (width 0.2) (layer "F.Cu") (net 1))
 (segment (start 53 87.213376) (end 50.118376 90.095) (width 0.2) (layer "F.Cu") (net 1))
 (segment (start 43.905 86.5) (end 39.5 86.5) (width 0.2) (layer "F.Cu") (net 1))
 (segment (start 47.5 90.095) (end 43.905 86.5) (width 0.2) (layer "F.Cu") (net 1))
 (segment (start 39.5 63) (end 39.5 86.5) (width 0.2) (layer "F.Cu") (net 1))
 (segment (start 53 87.075) (end 53 87.213376) (width 0.2) (layer "F.Cu") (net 1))
 (segment (start 44.149 58.351) (end 39.5 63) (width 0.2) (layer "B.Cu") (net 1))
 (segment (start 72.809 58.351) (end 44.149 58.351) (width 0.2) (layer "B.Cu") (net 1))
 (segment (start 75.66 55.5) (end 72.809 58.351) (width 0.2) (layer "B.Cu") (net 1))
 (segment (start 76 76.5) (end 76 83.5) (width 0.2) (layer "F.Cu") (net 6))
 (segment (start 74 74.5) (end 76 76.5) (width 0.2) (layer "F.Cu") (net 6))
 (segment (start 76 83.5) (end 74 85.5) (width 0.2) (layer "F.Cu") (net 6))
 (segment (start 75.0135 73.4865) (end 74 74.5) (width 0.2) (layer "F.Cu") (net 6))
 (segment (start 74 70) (end 75.0135 71.0135) (width 0.2) (layer "F.Cu") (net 6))
 (segment (start 75.0135 71.0135) (end 75.0135 73.4865) (width 0.2) (layer "F.Cu") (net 6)))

